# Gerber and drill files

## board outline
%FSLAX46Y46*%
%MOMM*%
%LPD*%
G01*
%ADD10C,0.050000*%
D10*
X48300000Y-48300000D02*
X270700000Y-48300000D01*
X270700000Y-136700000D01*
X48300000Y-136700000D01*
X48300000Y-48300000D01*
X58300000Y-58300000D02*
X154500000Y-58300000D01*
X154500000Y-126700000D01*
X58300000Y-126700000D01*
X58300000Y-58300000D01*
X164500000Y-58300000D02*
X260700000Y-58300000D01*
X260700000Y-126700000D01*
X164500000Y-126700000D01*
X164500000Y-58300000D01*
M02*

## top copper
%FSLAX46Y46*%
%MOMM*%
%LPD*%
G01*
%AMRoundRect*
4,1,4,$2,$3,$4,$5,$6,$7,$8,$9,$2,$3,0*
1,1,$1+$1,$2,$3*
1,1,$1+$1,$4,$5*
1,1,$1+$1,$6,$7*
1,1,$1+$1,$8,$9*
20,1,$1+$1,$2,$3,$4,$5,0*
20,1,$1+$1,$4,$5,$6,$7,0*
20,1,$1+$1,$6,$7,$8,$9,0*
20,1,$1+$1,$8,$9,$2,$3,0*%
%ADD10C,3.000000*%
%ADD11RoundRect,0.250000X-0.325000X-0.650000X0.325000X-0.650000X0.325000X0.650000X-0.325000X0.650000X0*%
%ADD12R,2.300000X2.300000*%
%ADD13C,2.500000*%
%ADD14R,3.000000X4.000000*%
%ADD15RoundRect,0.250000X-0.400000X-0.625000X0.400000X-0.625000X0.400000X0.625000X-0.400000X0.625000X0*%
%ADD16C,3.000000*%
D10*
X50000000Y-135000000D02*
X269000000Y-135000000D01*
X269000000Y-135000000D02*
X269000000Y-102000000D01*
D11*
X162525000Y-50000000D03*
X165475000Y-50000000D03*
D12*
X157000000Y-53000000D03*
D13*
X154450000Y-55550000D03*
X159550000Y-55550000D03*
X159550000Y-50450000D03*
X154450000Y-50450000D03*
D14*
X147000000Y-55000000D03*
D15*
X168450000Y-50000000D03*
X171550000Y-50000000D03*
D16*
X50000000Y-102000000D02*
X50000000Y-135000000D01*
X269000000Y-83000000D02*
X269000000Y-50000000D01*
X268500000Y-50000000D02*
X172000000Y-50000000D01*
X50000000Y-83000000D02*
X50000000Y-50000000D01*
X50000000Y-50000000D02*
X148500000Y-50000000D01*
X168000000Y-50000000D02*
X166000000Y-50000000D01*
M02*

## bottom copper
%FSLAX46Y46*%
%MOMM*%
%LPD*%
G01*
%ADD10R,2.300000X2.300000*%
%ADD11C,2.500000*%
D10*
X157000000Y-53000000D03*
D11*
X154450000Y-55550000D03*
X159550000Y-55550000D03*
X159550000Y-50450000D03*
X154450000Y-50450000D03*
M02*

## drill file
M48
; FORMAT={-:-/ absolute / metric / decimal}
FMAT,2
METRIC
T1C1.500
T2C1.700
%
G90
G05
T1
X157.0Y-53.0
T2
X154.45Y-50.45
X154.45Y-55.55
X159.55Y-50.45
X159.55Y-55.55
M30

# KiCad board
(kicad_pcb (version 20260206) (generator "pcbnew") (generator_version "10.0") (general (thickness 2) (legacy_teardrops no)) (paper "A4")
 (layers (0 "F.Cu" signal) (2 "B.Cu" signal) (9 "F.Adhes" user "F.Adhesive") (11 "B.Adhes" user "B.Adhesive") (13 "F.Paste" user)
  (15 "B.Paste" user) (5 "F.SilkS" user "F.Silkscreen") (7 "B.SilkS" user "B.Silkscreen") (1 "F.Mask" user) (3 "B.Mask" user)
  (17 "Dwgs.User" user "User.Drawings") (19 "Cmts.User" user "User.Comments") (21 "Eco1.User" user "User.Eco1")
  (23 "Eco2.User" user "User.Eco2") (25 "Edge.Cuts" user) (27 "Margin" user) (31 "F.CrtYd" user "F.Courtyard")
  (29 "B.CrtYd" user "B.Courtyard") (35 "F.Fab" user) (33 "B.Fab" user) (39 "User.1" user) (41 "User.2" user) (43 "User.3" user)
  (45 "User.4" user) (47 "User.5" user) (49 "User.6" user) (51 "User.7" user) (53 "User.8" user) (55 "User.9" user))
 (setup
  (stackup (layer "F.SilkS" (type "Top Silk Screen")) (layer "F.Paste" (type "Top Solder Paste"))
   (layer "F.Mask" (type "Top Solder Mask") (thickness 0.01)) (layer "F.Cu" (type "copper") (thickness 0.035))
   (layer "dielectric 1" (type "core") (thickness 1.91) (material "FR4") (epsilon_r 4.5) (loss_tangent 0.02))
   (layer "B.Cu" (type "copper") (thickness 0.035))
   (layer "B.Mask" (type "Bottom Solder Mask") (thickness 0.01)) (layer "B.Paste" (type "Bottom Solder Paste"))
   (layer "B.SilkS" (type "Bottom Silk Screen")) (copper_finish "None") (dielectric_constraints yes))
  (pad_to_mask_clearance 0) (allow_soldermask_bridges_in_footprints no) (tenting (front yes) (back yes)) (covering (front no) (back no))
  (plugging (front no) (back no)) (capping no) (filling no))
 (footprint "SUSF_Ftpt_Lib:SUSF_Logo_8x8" (layer "F.Cu") (at 150.5 130)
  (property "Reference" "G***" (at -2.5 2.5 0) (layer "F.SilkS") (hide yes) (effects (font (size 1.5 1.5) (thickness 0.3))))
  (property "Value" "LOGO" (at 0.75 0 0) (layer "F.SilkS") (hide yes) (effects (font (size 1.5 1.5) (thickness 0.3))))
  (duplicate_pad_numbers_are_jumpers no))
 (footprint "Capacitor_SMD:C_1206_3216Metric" (layer "F.Cu") (at 164 50)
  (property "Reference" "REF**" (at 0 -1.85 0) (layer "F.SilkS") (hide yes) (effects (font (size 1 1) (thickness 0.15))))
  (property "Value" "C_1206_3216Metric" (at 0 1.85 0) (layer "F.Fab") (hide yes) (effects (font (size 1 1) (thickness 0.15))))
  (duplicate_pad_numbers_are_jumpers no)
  (pad "1" smd roundrect (at -1.475 0) (size 1.15 1.8) (layers "F.Cu" "F.Mask" "F.Paste") (roundrect_rratio 0.217391) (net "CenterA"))
  (pad "2" smd roundrect (at 1.475 0) (size 1.15 1.8) (layers "F.Cu" "F.Mask" "F.Paste") (roundrect_rratio 0.217391) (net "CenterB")))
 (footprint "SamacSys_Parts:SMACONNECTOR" (layer "F.Cu") (at 157 53)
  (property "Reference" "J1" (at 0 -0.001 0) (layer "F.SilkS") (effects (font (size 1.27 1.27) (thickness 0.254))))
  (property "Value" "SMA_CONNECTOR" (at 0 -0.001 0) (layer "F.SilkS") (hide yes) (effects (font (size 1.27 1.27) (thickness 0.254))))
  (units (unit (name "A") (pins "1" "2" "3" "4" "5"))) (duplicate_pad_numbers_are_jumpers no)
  (pad "1" thru_hole rect (at 0 0) (size 2.3 2.3) (drill 1.5) (layers "*.Cu" "*.Mask") (remove_unused_layers no)
   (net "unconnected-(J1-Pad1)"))
  (pad "2" thru_hole circle (at -2.55 2.55) (size 2.5 2.5) (drill 1.7) (layers "*.Cu" "*.Mask") (remove_unused_layers no)
   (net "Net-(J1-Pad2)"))
  (pad "3" thru_hole circle (at 2.55 2.55) (size 2.5 2.5) (drill 1.7) (layers "*.Cu" "*.Mask") (remove_unused_layers no)
   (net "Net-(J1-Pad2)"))
  (pad "4" thru_hole circle (at 2.55 -2.55) (size 2.5 2.5) (drill 1.7) (layers "*.Cu" "*.Mask") (remove_unused_layers no)
   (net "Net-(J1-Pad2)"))
  (pad "5" thru_hole circle (at -2.55 -2.55) (size 2.5 2.5) (drill 1.7) (layers "*.Cu" "*.Mask") (remove_unused_layers no)
   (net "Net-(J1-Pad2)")))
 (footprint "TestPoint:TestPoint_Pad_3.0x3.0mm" (layer "F.Cu") (at 147 55)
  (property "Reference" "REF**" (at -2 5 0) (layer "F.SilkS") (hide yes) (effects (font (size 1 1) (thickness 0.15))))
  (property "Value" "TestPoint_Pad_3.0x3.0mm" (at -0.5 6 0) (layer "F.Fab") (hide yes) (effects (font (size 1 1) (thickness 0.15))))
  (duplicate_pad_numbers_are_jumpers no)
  (pad "2" smd rect (at 0 0) (size 3 4) (layers "F.Cu" "F.Mask") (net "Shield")))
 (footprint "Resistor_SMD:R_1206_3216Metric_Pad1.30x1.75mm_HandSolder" (layer "F.Cu") (at 170 50)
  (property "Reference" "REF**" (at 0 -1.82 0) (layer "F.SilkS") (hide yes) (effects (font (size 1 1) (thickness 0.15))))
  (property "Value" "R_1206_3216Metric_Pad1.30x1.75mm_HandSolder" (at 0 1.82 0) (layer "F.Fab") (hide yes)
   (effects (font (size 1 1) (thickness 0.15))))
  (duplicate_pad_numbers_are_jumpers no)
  (pad "1" smd roundrect (at -1.55 0) (size 1.3 1.75) (layers "F.Cu" "F.Mask" "F.Paste") (roundrect_rratio 0.192308) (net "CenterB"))
  (pad "2" smd roundrect (at 1.55 0) (size 1.3 1.75) (layers "F.Cu" "F.Mask" "F.Paste") (roundrect_rratio 0.192308) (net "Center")))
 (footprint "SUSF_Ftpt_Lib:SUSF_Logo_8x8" (layer "B.Cu") (at 168.336762 130 180)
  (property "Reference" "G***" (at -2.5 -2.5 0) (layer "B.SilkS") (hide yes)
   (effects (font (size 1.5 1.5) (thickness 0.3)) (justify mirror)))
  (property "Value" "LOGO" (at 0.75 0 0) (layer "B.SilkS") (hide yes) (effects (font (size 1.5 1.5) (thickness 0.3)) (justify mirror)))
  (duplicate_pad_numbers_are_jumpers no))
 (gr_line (start 50 135) (end 269 135) (stroke (width 3) (type default)) (layer "F.Cu"))
 (gr_line (start 269 135) (end 269 102) (stroke (width 3) (type default)) (layer "F.Cu"))
 (gr_rect (start 48.3 48.3) (end 270.7 136.7) (stroke (width 0.05) (type default)) (fill no) (layer "Edge.Cuts"))
 (gr_rect (start 58.3 58.3) (end 154.5 126.7) (stroke (width 0.05) (type default)) (fill no) (layer "Edge.Cuts"))
 (gr_rect (start 164.5 58.3) (end 260.7 126.7) (stroke (width 0.05) (type default)) (fill no) (layer "Edge.Cuts"))
 (segment (start 50 102) (end 50 135) (width 3) (layer "F.Cu") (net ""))
 (segment (start 269 83) (end 269 50) (width 3) (layer "F.Cu") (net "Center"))
 (segment (start 268.5 50) (end 172 50) (width 3) (layer "F.Cu") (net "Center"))
 (segment (start 50 83) (end 50 50) (width 3) (layer "F.Cu") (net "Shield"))
 (segment (start 50 50) (end 148.5 50) (width 3) (layer "F.Cu") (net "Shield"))
 (segment (start 168 50) (end 166 50) (width 3) (layer "F.Cu") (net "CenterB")))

